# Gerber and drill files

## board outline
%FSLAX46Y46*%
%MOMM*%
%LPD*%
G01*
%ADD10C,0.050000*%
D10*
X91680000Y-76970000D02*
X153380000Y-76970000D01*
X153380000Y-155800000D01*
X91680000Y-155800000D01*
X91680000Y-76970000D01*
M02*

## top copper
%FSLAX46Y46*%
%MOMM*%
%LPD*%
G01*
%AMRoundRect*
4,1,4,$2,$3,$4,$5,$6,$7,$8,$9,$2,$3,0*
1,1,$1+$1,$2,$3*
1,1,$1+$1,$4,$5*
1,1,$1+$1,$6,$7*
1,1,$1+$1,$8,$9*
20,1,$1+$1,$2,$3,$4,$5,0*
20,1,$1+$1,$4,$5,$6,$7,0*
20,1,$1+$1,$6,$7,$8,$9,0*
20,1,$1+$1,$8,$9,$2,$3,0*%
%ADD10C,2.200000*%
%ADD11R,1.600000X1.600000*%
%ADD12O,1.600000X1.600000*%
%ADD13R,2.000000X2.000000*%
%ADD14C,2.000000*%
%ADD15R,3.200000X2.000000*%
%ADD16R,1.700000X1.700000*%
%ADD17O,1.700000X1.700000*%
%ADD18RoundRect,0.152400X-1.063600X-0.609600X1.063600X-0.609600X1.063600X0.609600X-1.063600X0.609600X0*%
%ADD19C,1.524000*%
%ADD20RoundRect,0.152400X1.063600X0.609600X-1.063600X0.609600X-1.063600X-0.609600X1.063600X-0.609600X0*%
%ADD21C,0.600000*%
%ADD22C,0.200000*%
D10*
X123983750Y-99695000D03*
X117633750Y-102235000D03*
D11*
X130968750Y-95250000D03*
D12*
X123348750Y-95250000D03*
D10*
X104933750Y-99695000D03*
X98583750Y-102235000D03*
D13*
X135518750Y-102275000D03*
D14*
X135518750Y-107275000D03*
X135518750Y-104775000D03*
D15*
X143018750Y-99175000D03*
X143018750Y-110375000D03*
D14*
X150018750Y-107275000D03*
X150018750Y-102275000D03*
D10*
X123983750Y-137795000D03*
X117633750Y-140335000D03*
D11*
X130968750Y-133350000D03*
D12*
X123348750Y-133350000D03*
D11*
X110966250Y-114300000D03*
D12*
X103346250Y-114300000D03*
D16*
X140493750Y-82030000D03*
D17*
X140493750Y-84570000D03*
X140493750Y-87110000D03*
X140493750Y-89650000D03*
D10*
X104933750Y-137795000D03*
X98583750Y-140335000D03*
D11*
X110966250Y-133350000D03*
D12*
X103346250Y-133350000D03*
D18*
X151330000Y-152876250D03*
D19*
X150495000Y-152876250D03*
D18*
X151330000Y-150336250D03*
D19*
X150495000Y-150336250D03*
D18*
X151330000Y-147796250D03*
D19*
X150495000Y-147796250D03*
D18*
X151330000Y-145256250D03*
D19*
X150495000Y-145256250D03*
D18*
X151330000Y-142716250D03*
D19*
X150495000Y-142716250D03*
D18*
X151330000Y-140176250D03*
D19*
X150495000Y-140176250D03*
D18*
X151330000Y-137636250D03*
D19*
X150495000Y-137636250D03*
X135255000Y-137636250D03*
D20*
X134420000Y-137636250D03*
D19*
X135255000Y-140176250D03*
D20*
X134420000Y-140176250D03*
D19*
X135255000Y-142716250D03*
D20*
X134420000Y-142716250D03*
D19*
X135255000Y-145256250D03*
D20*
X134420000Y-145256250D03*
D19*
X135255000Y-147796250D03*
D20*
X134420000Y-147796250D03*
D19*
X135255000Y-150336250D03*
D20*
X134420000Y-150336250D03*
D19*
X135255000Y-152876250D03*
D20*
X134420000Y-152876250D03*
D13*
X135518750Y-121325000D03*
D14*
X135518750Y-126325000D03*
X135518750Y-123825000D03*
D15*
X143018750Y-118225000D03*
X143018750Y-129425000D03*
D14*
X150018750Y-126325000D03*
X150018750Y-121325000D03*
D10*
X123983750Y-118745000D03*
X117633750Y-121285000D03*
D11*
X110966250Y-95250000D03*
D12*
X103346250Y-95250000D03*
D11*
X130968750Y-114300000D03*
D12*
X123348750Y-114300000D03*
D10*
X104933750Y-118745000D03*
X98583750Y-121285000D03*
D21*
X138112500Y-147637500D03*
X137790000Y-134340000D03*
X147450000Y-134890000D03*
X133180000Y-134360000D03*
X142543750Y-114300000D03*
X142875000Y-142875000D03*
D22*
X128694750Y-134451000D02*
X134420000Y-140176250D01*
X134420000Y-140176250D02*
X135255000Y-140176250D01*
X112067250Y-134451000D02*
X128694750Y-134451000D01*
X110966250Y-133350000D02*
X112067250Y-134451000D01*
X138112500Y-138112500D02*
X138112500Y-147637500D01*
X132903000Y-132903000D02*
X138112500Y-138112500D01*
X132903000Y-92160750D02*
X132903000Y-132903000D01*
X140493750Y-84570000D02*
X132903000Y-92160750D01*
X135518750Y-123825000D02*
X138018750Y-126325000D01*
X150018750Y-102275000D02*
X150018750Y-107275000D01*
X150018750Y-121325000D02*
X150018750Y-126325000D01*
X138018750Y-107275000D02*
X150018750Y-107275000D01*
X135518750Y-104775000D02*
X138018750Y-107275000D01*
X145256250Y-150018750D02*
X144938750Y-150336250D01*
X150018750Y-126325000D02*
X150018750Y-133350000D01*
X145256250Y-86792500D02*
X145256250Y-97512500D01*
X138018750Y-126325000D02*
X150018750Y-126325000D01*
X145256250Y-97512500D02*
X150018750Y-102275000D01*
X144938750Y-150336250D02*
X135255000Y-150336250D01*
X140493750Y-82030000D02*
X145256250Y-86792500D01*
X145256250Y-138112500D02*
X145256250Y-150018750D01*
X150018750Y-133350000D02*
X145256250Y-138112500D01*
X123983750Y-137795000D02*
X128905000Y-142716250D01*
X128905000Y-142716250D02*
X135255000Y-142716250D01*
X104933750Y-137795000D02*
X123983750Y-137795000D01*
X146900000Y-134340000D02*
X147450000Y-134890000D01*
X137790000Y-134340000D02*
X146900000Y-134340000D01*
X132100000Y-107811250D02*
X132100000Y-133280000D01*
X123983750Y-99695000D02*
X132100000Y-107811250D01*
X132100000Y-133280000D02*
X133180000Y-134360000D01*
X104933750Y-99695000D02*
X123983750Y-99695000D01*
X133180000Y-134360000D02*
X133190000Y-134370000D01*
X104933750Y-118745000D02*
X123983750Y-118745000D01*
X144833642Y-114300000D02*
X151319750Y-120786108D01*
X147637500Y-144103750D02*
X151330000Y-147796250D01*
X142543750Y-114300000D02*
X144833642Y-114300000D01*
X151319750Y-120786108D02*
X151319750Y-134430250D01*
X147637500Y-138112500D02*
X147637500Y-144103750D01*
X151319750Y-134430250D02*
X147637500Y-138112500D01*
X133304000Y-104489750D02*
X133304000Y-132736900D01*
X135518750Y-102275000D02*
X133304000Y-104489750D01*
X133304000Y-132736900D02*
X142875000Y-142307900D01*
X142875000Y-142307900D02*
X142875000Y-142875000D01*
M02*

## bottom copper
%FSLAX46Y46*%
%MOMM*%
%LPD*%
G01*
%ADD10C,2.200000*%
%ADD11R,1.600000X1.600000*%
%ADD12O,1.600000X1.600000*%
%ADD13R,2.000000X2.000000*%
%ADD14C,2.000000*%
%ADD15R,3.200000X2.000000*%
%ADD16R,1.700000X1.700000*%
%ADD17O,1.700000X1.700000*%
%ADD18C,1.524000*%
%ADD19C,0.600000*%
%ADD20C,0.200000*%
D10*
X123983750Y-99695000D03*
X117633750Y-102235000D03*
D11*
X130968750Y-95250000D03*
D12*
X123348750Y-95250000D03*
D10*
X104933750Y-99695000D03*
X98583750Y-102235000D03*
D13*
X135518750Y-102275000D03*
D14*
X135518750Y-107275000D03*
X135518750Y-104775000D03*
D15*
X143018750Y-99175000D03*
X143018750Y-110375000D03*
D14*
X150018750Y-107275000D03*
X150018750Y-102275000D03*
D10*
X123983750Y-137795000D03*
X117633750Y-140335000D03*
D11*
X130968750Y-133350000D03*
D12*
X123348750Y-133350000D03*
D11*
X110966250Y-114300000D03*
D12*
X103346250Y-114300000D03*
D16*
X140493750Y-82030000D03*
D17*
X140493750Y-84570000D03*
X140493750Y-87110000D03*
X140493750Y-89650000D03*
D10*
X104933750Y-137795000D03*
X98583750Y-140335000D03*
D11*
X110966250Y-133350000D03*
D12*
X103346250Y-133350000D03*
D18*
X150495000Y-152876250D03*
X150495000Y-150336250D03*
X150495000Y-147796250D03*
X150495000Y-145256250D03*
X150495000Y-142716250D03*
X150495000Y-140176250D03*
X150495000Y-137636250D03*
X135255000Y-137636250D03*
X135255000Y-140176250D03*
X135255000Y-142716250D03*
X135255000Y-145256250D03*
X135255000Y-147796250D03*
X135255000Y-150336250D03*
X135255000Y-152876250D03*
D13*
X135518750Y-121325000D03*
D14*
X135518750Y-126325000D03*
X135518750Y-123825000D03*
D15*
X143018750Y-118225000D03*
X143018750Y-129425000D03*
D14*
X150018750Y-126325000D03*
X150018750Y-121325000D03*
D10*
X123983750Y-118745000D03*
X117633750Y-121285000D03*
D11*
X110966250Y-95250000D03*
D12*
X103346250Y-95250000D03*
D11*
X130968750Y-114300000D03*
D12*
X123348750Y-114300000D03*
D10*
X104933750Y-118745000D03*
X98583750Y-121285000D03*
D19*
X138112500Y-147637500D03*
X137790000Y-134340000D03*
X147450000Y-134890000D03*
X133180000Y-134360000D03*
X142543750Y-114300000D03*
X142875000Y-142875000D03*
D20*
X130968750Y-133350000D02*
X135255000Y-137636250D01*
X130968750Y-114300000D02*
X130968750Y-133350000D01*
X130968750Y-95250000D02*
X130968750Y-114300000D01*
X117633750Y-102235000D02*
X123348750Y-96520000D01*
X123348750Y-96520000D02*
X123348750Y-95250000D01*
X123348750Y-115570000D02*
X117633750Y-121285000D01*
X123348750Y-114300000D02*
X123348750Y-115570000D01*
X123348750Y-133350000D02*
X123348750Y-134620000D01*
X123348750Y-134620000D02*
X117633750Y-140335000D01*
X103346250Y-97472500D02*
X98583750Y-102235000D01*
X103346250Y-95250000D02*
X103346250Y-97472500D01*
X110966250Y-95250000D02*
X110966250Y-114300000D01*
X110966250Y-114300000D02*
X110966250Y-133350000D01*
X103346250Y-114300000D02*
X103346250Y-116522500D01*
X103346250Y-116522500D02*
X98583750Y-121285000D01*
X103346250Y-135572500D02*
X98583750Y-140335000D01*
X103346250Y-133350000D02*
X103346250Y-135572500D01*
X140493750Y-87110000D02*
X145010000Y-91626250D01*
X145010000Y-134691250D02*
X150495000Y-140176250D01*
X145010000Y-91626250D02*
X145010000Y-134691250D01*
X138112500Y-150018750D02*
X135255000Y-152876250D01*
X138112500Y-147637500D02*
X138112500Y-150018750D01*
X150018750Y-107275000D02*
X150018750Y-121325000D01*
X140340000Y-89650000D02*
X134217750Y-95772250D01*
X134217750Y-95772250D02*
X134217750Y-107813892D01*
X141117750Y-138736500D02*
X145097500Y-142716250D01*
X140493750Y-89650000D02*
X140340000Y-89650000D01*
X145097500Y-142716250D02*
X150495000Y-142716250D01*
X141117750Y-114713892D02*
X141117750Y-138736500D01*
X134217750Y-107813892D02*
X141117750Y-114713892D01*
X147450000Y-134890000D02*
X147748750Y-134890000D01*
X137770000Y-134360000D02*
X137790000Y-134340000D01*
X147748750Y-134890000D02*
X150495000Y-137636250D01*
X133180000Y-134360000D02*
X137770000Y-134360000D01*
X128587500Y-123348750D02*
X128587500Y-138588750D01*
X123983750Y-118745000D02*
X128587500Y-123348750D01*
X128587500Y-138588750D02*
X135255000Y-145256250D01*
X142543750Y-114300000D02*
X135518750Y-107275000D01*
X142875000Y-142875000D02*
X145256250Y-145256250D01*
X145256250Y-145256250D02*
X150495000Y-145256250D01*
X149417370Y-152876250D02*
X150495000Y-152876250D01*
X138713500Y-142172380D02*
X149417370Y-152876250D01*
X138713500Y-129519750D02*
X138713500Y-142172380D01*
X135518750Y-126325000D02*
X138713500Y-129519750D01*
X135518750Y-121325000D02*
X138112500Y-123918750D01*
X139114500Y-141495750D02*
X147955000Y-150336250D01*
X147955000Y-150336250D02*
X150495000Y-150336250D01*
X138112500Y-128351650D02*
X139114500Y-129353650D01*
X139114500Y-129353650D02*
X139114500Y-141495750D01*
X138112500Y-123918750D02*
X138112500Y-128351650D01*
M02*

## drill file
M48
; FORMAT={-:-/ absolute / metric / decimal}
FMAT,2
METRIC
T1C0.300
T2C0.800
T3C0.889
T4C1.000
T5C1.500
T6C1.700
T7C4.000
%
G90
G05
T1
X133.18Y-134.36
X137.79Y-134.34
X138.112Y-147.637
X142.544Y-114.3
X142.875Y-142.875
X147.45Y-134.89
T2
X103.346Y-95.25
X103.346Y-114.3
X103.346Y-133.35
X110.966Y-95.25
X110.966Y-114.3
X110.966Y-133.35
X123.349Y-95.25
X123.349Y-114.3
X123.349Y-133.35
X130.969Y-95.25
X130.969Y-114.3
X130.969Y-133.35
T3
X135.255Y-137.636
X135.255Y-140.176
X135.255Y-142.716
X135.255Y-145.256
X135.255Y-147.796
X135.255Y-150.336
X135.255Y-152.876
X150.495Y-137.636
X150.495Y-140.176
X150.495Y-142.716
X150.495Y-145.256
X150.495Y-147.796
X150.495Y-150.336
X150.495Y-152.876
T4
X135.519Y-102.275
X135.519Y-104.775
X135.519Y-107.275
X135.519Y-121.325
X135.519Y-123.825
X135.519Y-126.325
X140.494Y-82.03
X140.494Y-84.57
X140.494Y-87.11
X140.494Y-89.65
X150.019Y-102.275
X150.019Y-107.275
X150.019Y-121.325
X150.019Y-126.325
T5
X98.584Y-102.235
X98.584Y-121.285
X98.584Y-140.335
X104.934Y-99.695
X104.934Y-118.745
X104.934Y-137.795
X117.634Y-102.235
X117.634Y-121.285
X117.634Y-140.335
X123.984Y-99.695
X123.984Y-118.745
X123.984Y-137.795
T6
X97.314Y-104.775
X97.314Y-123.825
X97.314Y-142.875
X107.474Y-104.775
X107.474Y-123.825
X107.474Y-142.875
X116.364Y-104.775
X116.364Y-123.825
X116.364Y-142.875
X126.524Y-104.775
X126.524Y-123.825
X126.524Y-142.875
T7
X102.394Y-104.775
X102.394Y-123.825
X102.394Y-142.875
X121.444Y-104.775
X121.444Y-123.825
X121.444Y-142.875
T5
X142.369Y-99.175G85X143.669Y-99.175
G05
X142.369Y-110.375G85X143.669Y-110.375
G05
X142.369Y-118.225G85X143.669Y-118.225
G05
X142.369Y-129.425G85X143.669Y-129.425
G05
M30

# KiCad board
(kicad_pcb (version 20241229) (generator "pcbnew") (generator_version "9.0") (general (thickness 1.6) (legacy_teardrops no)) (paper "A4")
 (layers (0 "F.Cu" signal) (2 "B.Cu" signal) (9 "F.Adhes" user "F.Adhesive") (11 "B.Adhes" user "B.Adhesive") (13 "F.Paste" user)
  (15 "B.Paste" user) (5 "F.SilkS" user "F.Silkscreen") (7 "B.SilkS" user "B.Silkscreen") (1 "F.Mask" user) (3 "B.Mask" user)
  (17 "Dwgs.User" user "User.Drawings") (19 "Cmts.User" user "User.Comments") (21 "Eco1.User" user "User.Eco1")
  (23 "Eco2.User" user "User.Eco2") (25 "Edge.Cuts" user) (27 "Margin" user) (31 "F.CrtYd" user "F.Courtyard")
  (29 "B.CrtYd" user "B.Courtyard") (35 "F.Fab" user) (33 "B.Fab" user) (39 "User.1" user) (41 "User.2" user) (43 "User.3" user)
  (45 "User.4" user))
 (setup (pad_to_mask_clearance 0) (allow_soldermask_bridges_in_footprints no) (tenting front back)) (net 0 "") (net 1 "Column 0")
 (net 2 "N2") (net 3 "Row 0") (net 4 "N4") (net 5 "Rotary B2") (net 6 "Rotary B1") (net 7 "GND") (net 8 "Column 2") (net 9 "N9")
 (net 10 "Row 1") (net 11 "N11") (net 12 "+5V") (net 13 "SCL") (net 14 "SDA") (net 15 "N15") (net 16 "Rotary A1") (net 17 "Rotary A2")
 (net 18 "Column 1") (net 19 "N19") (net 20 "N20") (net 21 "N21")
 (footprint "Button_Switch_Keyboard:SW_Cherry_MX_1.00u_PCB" (layer "F.Cu") (at 123.98375 99.695)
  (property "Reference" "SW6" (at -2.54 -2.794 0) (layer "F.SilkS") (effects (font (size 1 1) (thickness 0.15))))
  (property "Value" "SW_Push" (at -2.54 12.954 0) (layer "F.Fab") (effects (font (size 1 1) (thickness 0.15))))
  (pad "" np_thru_hole circle (at -7.62 5.08) (size 1.7 1.7) (drill 1.7) (layers "*.Cu" "*.Mask"))
  (pad "" np_thru_hole circle (at -2.54 5.08) (size 4 4) (drill 4) (layers "*.Cu" "*.Mask"))
  (pad "" np_thru_hole circle (at 2.54 5.08) (size 1.7 1.7) (drill 1.7) (layers "*.Cu" "*.Mask"))
  (pad "1" thru_hole circle (at 0 0) (size 2.2 2.2) (drill 1.5) (layers "*.Cu" "*.Mask") (remove_unused_layers no) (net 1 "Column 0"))
  (pad "2" thru_hole circle (at -6.35 2.54) (size 2.2 2.2) (drill 1.5) (layers "*.Cu" "*.Mask") (remove_unused_layers no) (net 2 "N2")))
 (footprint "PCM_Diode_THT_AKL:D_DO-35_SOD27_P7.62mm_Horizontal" (layer "F.Cu") (at 130.96875 95.25 180)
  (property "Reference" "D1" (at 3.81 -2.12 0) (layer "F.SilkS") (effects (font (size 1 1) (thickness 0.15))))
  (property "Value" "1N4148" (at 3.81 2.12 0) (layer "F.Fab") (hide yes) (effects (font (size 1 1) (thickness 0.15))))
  (pad "1" thru_hole rect (at 0 0 180) (size 1.6 1.6) (drill 0.8) (layers "*.Cu" "*.Mask") (remove_unused_layers no) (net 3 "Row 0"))
  (pad "2" thru_hole oval (at 7.62 0 180) (size 1.6 1.6) (drill 0.8) (layers "*.Cu" "*.Mask") (remove_unused_layers no) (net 2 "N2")))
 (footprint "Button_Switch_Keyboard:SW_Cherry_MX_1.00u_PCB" (layer "F.Cu") (at 104.93375 99.695)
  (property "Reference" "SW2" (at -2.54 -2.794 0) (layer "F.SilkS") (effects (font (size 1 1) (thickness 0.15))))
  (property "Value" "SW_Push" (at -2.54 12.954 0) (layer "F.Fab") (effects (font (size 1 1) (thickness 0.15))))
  (pad "" np_thru_hole circle (at -7.62 5.08) (size 1.7 1.7) (drill 1.7) (layers "*.Cu" "*.Mask"))
  (pad "" np_thru_hole circle (at -2.54 5.08) (size 4 4) (drill 4) (layers "*.Cu" "*.Mask"))
  (pad "" np_thru_hole circle (at 2.54 5.08) (size 1.7 1.7) (drill 1.7) (layers "*.Cu" "*.Mask"))
  (pad "1" thru_hole circle (at 0 0) (size 2.2 2.2) (drill 1.5) (layers "*.Cu" "*.Mask") (remove_unused_layers no) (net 1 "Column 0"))
  (pad "2" thru_hole circle (at -6.35 2.54) (size 2.2 2.2) (drill 1.5) (layers "*.Cu" "*.Mask") (remove_unused_layers no) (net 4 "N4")))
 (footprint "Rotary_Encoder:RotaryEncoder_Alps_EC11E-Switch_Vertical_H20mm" (layer "F.Cu") (at 135.51875 102.275)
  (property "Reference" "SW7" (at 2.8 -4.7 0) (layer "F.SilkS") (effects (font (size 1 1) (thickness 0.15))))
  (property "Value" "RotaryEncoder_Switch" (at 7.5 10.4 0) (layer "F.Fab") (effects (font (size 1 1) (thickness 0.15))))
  (pad "A" thru_hole rect (at 0 0) (size 2 2) (drill 1) (layers "*.Cu" "*.Mask") (remove_unused_layers no) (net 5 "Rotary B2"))
  (pad "B" thru_hole circle (at 0 5) (size 2 2) (drill 1) (layers "*.Cu" "*.Mask") (remove_unused_layers no) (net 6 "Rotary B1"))
  (pad "C" thru_hole circle (at 0 2.5) (size 2 2) (drill 1) (layers "*.Cu" "*.Mask") (remove_unused_layers no) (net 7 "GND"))
  (pad "MP" thru_hole rect (at 7.5 -3.1) (size 3.2 2) (drill oval 2.8 1.5) (layers "*.Cu" "*.Mask") (remove_unused_layers no))
  (pad "MP" thru_hole rect (at 7.5 8.1) (size 3.2 2) (drill oval 2.8 1.5) (layers "*.Cu" "*.Mask") (remove_unused_layers no))
  (pad "S1" thru_hole circle (at 14.5 5) (size 2 2) (drill 1) (layers "*.Cu" "*.Mask") (remove_unused_layers no) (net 7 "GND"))
  (pad "S2" thru_hole circle (at 14.5 0) (size 2 2) (drill 1) (layers "*.Cu" "*.Mask") (remove_unused_layers no) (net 7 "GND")))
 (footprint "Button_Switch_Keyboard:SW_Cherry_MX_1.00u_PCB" (layer "F.Cu") (at 123.98375 137.795)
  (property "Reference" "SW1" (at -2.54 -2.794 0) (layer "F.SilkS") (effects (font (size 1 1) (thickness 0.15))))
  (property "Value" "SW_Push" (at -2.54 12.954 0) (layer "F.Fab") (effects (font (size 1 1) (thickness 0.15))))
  (pad "" np_thru_hole circle (at -7.62 5.08) (size 1.7 1.7) (drill 1.7) (layers "*.Cu" "*.Mask"))
  (pad "" np_thru_hole circle (at -2.54 5.08) (size 4 4) (drill 4) (layers "*.Cu" "*.Mask"))
  (pad "" np_thru_hole circle (at 2.54 5.08) (size 1.7 1.7) (drill 1.7) (layers "*.Cu" "*.Mask"))
  (pad "1" thru_hole circle (at 0 0) (size 2.2 2.2) (drill 1.5) (layers "*.Cu" "*.Mask") (remove_unused_layers no) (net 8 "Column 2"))
  (pad "2" thru_hole circle (at -6.35 2.54) (size 2.2 2.2) (drill 1.5) (layers "*.Cu" "*.Mask") (remove_unused_layers no) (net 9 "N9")))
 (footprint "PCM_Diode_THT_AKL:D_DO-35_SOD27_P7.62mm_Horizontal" (layer "F.Cu") (at 130.96875 133.35 180)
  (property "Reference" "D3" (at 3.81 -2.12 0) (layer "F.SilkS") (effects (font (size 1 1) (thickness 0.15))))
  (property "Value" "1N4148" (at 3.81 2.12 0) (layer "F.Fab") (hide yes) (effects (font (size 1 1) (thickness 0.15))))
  (pad "1" thru_hole rect (at 0 0 180) (size 1.6 1.6) (drill 0.8) (layers "*.Cu" "*.Mask") (remove_unused_layers no) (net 3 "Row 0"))
  (pad "2" thru_hole oval (at 7.62 0 180) (size 1.6 1.6) (drill 0.8) (layers "*.Cu" "*.Mask") (remove_unused_layers no) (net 9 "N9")))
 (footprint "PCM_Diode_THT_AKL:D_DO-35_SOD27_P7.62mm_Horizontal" (layer "F.Cu") (at 110.96625 114.3 180)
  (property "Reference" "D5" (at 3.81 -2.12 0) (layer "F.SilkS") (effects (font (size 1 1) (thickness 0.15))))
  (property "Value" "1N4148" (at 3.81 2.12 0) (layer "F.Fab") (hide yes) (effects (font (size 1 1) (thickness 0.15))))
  (pad "1" thru_hole rect (at 0 0 180) (size 1.6 1.6) (drill 0.8) (layers "*.Cu" "*.Mask") (remove_unused_layers no) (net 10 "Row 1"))
  (pad "2" thru_hole oval (at 7.62 0 180) (size 1.6 1.6) (drill 0.8) (layers "*.Cu" "*.Mask") (remove_unused_layers no) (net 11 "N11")))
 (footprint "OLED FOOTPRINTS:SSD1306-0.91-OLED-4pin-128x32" (layer "F.Cu") (at 103.99375 79.84)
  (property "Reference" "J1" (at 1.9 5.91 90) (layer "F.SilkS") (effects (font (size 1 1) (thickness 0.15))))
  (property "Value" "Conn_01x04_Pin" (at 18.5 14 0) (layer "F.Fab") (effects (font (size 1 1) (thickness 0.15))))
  (pad "1" thru_hole rect (at 36.5 2.19) (size 1.7 1.7) (drill 1) (layers "*.Cu" "*.Mask") (remove_unused_layers no) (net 7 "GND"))
  (pad "2" thru_hole oval (at 36.5 4.73) (size 1.7 1.7) (drill 1) (layers "*.Cu" "*.Mask") (remove_unused_layers no) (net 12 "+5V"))
  (pad "3" thru_hole oval (at 36.5 7.27) (size 1.7 1.7) (drill 1) (layers "*.Cu" "*.Mask") (remove_unused_layers no) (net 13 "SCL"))
  (pad "4" thru_hole oval (at 36.5 9.81) (size 1.7 1.7) (drill 1) (layers "*.Cu" "*.Mask") (remove_unused_layers no) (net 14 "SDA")))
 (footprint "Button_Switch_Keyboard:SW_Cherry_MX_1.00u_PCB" (layer "F.Cu") (at 104.93375 137.795)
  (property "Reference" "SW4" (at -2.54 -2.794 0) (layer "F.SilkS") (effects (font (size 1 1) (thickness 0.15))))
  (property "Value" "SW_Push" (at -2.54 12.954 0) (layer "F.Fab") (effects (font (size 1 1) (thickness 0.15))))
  (pad "" np_thru_hole circle (at -7.62 5.08) (size 1.7 1.7) (drill 1.7) (layers "*.Cu" "*.Mask"))
  (pad "" np_thru_hole circle (at -2.54 5.08) (size 4 4) (drill 4) (layers "*.Cu" "*.Mask"))
  (pad "" np_thru_hole circle (at 2.54 5.08) (size 1.7 1.7) (drill 1.7) (layers "*.Cu" "*.Mask"))
  (pad "1" thru_hole circle (at 0 0) (size 2.2 2.2) (drill 1.5) (layers "*.Cu" "*.Mask") (remove_unused_layers no) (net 8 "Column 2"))
  (pad "2" thru_hole circle (at -6.35 2.54) (size 2.2 2.2) (drill 1.5) (layers "*.Cu" "*.Mask") (remove_unused_layers no) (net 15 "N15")))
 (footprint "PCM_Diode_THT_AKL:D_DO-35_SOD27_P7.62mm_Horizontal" (layer "F.Cu") (at 110.96625 133.35 180)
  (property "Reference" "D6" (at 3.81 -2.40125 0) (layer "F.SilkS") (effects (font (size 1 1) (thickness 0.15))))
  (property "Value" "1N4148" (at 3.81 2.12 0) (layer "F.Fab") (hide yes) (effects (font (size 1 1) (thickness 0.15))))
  (pad "1" thru_hole rect (at 0 0 180) (size 1.6 1.6) (drill 0.8) (layers "*.Cu" "*.Mask") (remove_unused_layers no) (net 10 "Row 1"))
  (pad "2" thru_hole oval (at 7.62 0 180) (size 1.6 1.6) (drill 0.8) (layers "*.Cu" "*.Mask") (remove_unused_layers no) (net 15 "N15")))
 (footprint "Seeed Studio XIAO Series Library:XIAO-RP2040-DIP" (layer "F.Cu") (at 142.875 145.25625 180)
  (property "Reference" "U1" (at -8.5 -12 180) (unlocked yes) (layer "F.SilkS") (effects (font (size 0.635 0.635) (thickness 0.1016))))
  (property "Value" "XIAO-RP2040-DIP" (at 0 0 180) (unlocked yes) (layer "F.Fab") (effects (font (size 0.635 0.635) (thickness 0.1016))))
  (pad "1" smd roundrect (at -8.455 -7.62) (size 2.432 1.524) (layers "F.Cu" "F.Mask") (roundrect_rratio 0.1) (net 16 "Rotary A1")
   (thermal_bridge_angle 45))
  (pad "1" thru_hole circle (at -7.62 -7.62) (size 1.524 1.524) (drill 0.889) (layers "*.Cu" "*.Mask") (remove_unused_layers no)
   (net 16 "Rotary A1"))
  (pad "2" smd roundrect (at -8.455 -5.08) (size 2.432 1.524) (layers "F.Cu" "F.Mask") (roundrect_rratio 0.1) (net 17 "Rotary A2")
   (thermal_bridge_angle 45))
  (pad "2" thru_hole circle (at -7.62 -5.08) (size 1.524 1.524) (drill 0.889) (layers "*.Cu" "*.Mask") (remove_unused_layers no)
   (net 17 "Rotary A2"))
  (pad "3" smd roundrect (at -8.455 -2.54) (size 2.432 1.524) (layers "F.Cu" "F.Mask") (roundrect_rratio 0.1) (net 6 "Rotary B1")
   (thermal_bridge_angle 45))
  (pad "3" thru_hole circle (at -7.62 -2.54) (size 1.524 1.524) (drill 0.889) (layers "*.Cu" "*.Mask") (remove_unused_layers no)
   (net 6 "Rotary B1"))
  (pad "4" smd roundrect (at -8.455 0) (size 2.432 1.524) (layers "F.Cu" "F.Mask") (roundrect_rratio 0.1) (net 5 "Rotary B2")
   (thermal_bridge_angle 45))
  (pad "4" thru_hole circle (at -7.62 0) (size 1.524 1.524) (drill 0.889) (layers "*.Cu" "*.Mask") (remove_unused_layers no)
   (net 5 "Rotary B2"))
  (pad "5" smd roundrect (at -8.455 2.54) (size 2.432 1.524) (layers "F.Cu" "F.Mask") (roundrect_rratio 0.1) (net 14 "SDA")
   (thermal_bridge_angle 45))
  (pad "5" thru_hole circle (at -7.62 2.54) (size 1.524 1.524) (drill 0.889) (layers "*.Cu" "*.Mask") (remove_unused_layers no)
   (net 14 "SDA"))
  (pad "6" smd roundrect (at -8.455 5.08) (size 2.432 1.524) (layers "F.Cu" "F.Mask") (roundrect_rratio 0.1) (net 13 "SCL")
   (thermal_bridge_angle 45))
  (pad "6" thru_hole circle (at -7.62 5.08) (size 1.524 1.524) (drill 0.889) (layers "*.Cu" "*.Mask") (remove_unused_layers no)
   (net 13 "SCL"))
  (pad "7" smd roundrect (at -8.455 7.62) (size 2.432 1.524) (layers "F.Cu" "F.Mask") (roundrect_rratio 0.1) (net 1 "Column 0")
   (thermal_bridge_angle 45))
  (pad "7" thru_hole circle (at -7.62 7.62) (size 1.524 1.524) (drill 0.889) (layers "*.Cu" "*.Mask") (remove_unused_layers no)
   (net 1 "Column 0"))
  (pad "8" thru_hole circle (at 7.62 7.62 180) (size 1.524 1.524) (drill 0.889) (layers "*.Cu" "*.Mask") (remove_unused_layers no)
   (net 3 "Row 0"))
  (pad "8" smd roundrect (at 8.455 7.62 180) (size 2.432 1.524) (layers "F.Cu" "F.Mask") (roundrect_rratio 0.1) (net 3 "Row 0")
   (thermal_bridge_angle 45))
  (pad "9" thru_hole circle (at 7.62 5.08 180) (size 1.524 1.524) (drill 0.889) (layers "*.Cu" "*.Mask") (remove_unused_layers no)
   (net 10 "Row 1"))
  (pad "9" smd roundrect (at 8.455 5.08 180) (size 2.432 1.524) (layers "F.Cu" "F.Mask") (roundrect_rratio 0.1) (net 10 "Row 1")
   (thermal_bridge_angle 45))
  (pad "10" thru_hole circle (at 7.62 2.54 180) (size 1.524 1.524) (drill 0.889) (layers "*.Cu" "*.Mask") (remove_unused_layers no)
   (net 8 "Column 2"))
  (pad "10" smd roundrect (at 8.455 2.54 180) (size 2.432 1.524) (layers "F.Cu" "F.Mask") (roundrect_rratio 0.1) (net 8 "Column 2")
   (thermal_bridge_angle 45))
  (pad "11" thru_hole circle (at 7.62 0 180) (size 1.524 1.524) (drill 0.889) (layers "*.Cu" "*.Mask") (remove_unused_layers no)
   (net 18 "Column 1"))
  (pad "11" smd roundrect (at 8.455 0 180) (size 2.432 1.524) (layers "F.Cu" "F.Mask") (roundrect_rratio 0.1) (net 18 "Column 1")
   (thermal_bridge_angle 45))
  (pad "12" thru_hole circle (at 7.62 -2.54 180) (size 1.524 1.524) (drill 0.889) (layers "*.Cu" "*.Mask") (remove_unused_layers no)
   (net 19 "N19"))
  (pad "12" smd roundrect (at 8.455 -2.54 180) (size 2.432 1.524) (layers "F.Cu" "F.Mask") (roundrect_rratio 0.1) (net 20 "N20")
   (thermal_bridge_angle 45))
  (pad "13" thru_hole circle (at 7.62 -5.08 180) (size 1.524 1.524) (drill 0.889) (layers "*.Cu" "*.Mask") (remove_unused_layers no)
   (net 7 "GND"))
  (pad "13" smd roundrect (at 8.455 -5.08 180) (size 2.432 1.524) (layers "F.Cu" "F.Mask") (roundrect_rratio 0.1) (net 7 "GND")
   (thermal_bridge_angle 45))
  (pad "14" thru_hole circle (at 7.62 -7.62 180) (size 1.524 1.524) (drill 0.889) (layers "*.Cu" "*.Mask") (remove_unused_layers no)
   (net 12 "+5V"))
  (pad "14" smd roundrect (at 8.455 -7.62 180) (size 2.432 1.524) (layers "F.Cu" "F.Mask") (roundrect_rratio 0.1) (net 12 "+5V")
   (thermal_bridge_angle 45)))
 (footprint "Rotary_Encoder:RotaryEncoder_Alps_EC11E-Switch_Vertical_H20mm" (layer "F.Cu") (at 135.51875 121.325)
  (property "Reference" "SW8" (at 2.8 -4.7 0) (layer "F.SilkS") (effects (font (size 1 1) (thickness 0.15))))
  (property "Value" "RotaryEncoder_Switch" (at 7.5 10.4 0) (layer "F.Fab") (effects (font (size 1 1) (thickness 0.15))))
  (pad "A" thru_hole rect (at 0 0) (size 2 2) (drill 1) (layers "*.Cu" "*.Mask") (remove_unused_layers no) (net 17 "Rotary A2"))
  (pad "B" thru_hole circle (at 0 5) (size 2 2) (drill 1) (layers "*.Cu" "*.Mask") (remove_unused_layers no) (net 16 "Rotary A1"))
  (pad "C" thru_hole circle (at 0 2.5) (size 2 2) (drill 1) (layers "*.Cu" "*.Mask") (remove_unused_layers no) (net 7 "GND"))
  (pad "MP" thru_hole rect (at 7.5 -3.1) (size 3.2 2) (drill oval 2.8 1.5) (layers "*.Cu" "*.Mask") (remove_unused_layers no))
  (pad "MP" thru_hole rect (at 7.5 8.1) (size 3.2 2) (drill oval 2.8 1.5) (layers "*.Cu" "*.Mask") (remove_unused_layers no))
  (pad "S1" thru_hole circle (at 14.5 5) (size 2 2) (drill 1) (layers "*.Cu" "*.Mask") (remove_unused_layers no) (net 7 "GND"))
  (pad "S2" thru_hole circle (at 14.5 0) (size 2 2) (drill 1) (layers "*.Cu" "*.Mask") (remove_unused_layers no) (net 7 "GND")))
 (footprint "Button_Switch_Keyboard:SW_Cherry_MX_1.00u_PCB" (layer "F.Cu") (at 123.98375 118.745)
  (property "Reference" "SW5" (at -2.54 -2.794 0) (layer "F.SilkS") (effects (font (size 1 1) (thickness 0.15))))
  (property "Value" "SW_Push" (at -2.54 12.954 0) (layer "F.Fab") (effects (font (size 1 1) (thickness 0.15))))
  (pad "" np_thru_hole circle (at -7.62 5.08) (size 1.7 1.7) (drill 1.7) (layers "*.Cu" "*.Mask"))
  (pad "" np_thru_hole circle (at -2.54 5.08) (size 4 4) (drill 4) (layers "*.Cu" "*.Mask"))
  (pad "" np_thru_hole circle (at 2.54 5.08) (size 1.7 1.7) (drill 1.7) (layers "*.Cu" "*.Mask"))
  (pad "1" thru_hole circle (at 0 0) (size 2.2 2.2) (drill 1.5) (layers "*.Cu" "*.Mask") (remove_unused_layers no) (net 18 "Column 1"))
  (pad "2" thru_hole circle (at -6.35 2.54) (size 2.2 2.2) (drill 1.5) (layers "*.Cu" "*.Mask") (remove_unused_layers no) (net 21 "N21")))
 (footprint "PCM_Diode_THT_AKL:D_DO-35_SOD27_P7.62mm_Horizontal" (layer "F.Cu") (at 110.96625 95.25 180)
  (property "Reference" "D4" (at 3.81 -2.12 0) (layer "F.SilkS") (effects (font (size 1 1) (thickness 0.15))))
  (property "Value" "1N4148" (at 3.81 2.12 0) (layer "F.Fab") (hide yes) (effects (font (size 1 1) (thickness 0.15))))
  (pad "1" thru_hole rect (at 0 0 180) (size 1.6 1.6) (drill 0.8) (layers "*.Cu" "*.Mask") (remove_unused_layers no) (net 10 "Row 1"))
  (pad "2" thru_hole oval (at 7.62 0 180) (size 1.6 1.6) (drill 0.8) (layers "*.Cu" "*.Mask") (remove_unused_layers no) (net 4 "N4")))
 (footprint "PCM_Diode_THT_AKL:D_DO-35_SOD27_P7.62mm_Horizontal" (layer "F.Cu") (at 130.96875 114.3 180)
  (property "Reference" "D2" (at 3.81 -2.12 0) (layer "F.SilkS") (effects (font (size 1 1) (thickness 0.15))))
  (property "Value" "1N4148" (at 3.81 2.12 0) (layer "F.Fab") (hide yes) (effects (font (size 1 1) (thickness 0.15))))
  (pad "1" thru_hole rect (at 0 0 180) (size 1.6 1.6) (drill 0.8) (layers "*.Cu" "*.Mask") (remove_unused_layers no) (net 3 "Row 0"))
  (pad "2" thru_hole oval (at 7.62 0 180) (size 1.6 1.6) (drill 0.8) (layers "*.Cu" "*.Mask") (remove_unused_layers no) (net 21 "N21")))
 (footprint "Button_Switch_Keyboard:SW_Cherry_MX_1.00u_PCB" (layer "F.Cu") (at 104.93375 118.745)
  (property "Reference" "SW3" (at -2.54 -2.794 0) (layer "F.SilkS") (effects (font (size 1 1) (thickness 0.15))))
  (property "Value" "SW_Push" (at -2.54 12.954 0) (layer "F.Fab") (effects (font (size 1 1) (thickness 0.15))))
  (pad "" np_thru_hole circle (at -7.62 5.08) (size 1.7 1.7) (drill 1.7) (layers "*.Cu" "*.Mask"))
  (pad "" np_thru_hole circle (at -2.54 5.08) (size 4 4) (drill 4) (layers "*.Cu" "*.Mask"))
  (pad "" np_thru_hole circle (at 2.54 5.08) (size 1.7 1.7) (drill 1.7) (layers "*.Cu" "*.Mask"))
  (pad "1" thru_hole circle (at 0 0) (size 2.2 2.2) (drill 1.5) (layers "*.Cu" "*.Mask") (remove_unused_layers no) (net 18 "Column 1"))
  (pad "2" thru_hole circle (at -6.35 2.54) (size 2.2 2.2) (drill 1.5) (layers "*.Cu" "*.Mask") (remove_unused_layers no) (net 11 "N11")))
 (gr_rect (start 91.68 76.97) (end 153.38 155.8) (stroke (width 0.05) (type default)) (fill no) (layer "Edge.Cuts"))
 (segment (start 130.96875 133.35) (end 135.255 137.63625) (width 0.2) (layer "B.Cu") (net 3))
 (segment (start 130.96875 114.3) (end 130.96875 133.35) (width 0.2) (layer "B.Cu") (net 3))
 (segment (start 130.96875 95.25) (end 130.96875 114.3) (width 0.2) (layer "B.Cu") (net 3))
 (segment (start 117.63375 102.235) (end 123.34875 96.52) (width 0.2) (layer "B.Cu") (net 2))
 (segment (start 123.34875 96.52) (end 123.34875 95.25) (width 0.2) (layer "B.Cu") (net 2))
 (segment (start 123.34875 115.57) (end 117.63375 121.285) (width 0.2) (layer "B.Cu") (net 21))
 (segment (start 123.34875 114.3) (end 123.34875 115.57) (width 0.2) (layer "B.Cu") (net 21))
 (segment (start 123.34875 133.35) (end 123.34875 134.62) (width 0.2) (layer "B.Cu") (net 9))
 (segment (start 123.34875 134.62) (end 117.63375 140.335) (width 0.2) (layer "B.Cu") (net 9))
 (segment (start 103.34625 97.4725) (end 98.58375 102.235) (width 0.2) (layer "B.Cu") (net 4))
 (segment (start 103.34625 95.25) (end 103.34625 97.4725) (width 0.2) (layer "B.Cu") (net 4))
 (segment (start 128.69475 134.451) (end 134.42 140.17625) (width 0.2) (layer "F.Cu") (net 10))
 (segment (start 134.42 140.17625) (end 135.255 140.17625) (width 0.2) (layer "F.Cu") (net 10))
 (segment (start 112.06725 134.451) (end 128.69475 134.451) (width 0.2) (layer "F.Cu") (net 10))
 (segment (start 110.96625 133.35) (end 112.06725 134.451) (width 0.2) (layer "F.Cu") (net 10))
 (segment (start 110.96625 95.25) (end 110.96625 114.3) (width 0.2) (layer "B.Cu") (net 10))
 (segment (start 110.96625 114.3) (end 110.96625 133.35) (width 0.2) (layer "B.Cu") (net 10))
 (segment (start 103.34625 114.3) (end 103.34625 116.5225) (width 0.2) (layer "B.Cu") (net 11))
 (segment (start 103.34625 116.5225) (end 98.58375 121.285) (width 0.2) (layer "B.Cu") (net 11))
 (segment (start 103.34625 135.5725) (end 98.58375 140.335) (width 0.2) (layer "B.Cu") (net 15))
 (segment (start 103.34625 133.35) (end 103.34625 135.5725) (width 0.2) (layer "B.Cu") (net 15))
 (segment (start 140.49375 87.11) (end 145.01 91.62625) (width 0.2) (layer "B.Cu") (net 13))
 (segment (start 145.01 134.69125) (end 150.495 140.17625) (width 0.2) (layer "B.Cu") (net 13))
 (segment (start 145.01 91.62625) (end 145.01 134.69125) (width 0.2) (layer "B.Cu") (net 13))
 (segment (start 138.1125 138.1125) (end 138.1125 147.6375) (width 0.2) (layer "F.Cu") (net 12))
 (segment (start 132.903 132.903) (end 138.1125 138.1125) (width 0.2) (layer "F.Cu") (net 12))
 (segment (start 132.903 92.16075) (end 132.903 132.903) (width 0.2) (layer "F.Cu") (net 12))
 (segment (start 140.49375 84.57) (end 132.903 92.16075) (width 0.2) (layer "F.Cu") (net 12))
 (via (at 138.1125 147.6375) (size 0.6) (drill 0.3) (layers "F.Cu" "B.Cu") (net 12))
 (segment (start 138.1125 150.01875) (end 135.255 152.87625) (width 0.2) (layer "B.Cu") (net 12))
 (segment (start 138.1125 147.6375) (end 138.1125 150.01875) (width 0.2) (layer "B.Cu") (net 12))
 (segment (start 135.51875 123.825) (end 138.01875 126.325) (width 0.2) (layer "F.Cu") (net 7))
 (segment (start 150.01875 102.275) (end 150.01875 107.275) (width 0.2) (layer "F.Cu") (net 7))
 (segment (start 150.01875 121.325) (end 150.01875 126.325) (width 0.2) (layer "F.Cu") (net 7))
 (segment (start 138.01875 107.275) (end 150.01875 107.275) (width 0.2) (layer "F.Cu") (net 7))
 (segment (start 135.51875 104.775) (end 138.01875 107.275) (width 0.2) (layer "F.Cu") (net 7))
 (segment (start 145.25625 150.01875) (end 144.93875 150.33625) (width 0.2) (layer "F.Cu") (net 7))
 (segment (start 150.01875 126.325) (end 150.01875 133.35) (width 0.2) (layer "F.Cu") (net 7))
 (segment (start 145.25625 86.7925) (end 145.25625 97.5125) (width 0.2) (layer "F.Cu") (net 7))
 (segment (start 138.01875 126.325) (end 150.01875 126.325) (width 0.2) (layer "F.Cu") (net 7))
 (segment (start 145.25625 97.5125) (end 150.01875 102.275) (width 0.2) (layer "F.Cu") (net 7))
 (segment (start 144.93875 150.33625) (end 135.255 150.33625) (width 0.2) (layer "F.Cu") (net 7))
 (segment (start 140.49375 82.03) (end 145.25625 86.7925) (width 0.2) (layer "F.Cu") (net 7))
 (segment (start 145.25625 138.1125) (end 145.25625 150.01875) (width 0.2) (layer "F.Cu") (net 7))
 (segment (start 150.01875 133.35) (end 145.25625 138.1125) (width 0.2) (layer "F.Cu") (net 7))
 (segment (start 150.01875 107.275) (end 150.01875 121.325) (width 0.2) (layer "B.Cu") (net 7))
 (segment (start 140.34 89.65) (end 134.21775 95.77225) (width 0.2) (layer "B.Cu") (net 14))
 (segment (start 134.21775 95.77225) (end 134.21775 107.813892) (width 0.2) (layer "B.Cu") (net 14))
 (segment (start 141.11775 138.7365) (end 145.0975 142.71625) (width 0.2) (layer "B.Cu") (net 14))
 (segment (start 140.49375 89.65) (end 140.34 89.65) (width 0.2) (layer "B.Cu") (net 14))
 (segment (start 145.0975 142.71625) (end 150.495 142.71625) (width 0.2) (layer "B.Cu") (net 14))
 (segment (start 141.11775 114.713892) (end 141.11775 138.7365) (width 0.2) (layer "B.Cu") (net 14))
 (segment (start 134.21775 107.813892) (end 141.11775 114.713892) (width 0.2) (layer "B.Cu") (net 14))
 (segment (start 123.98375 137.795) (end 128.905 142.71625) (width 0.2) (layer "F.Cu") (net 8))
 (segment (start 128.905 142.71625) (end 135.255 142.71625) (width 0.2) (layer "F.Cu") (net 8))
 (segment (start 104.93375 137.795) (end 123.98375 137.795) (width 0.2) (layer "F.Cu") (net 8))
 (segment (start 146.9 134.34) (end 147.45 134.89) (width 0.2) (layer "F.Cu") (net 1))
 (segment (start 137.79 134.34) (end 146.9 134.34) (width 0.2) (layer "F.Cu") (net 1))
 (segment (start 132.1 107.81125) (end 132.1 133.28) (width 0.2) (layer "F.Cu") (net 1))
 (segment (start 123.98375 99.695) (end 132.1 107.81125) (width 0.2) (layer "F.Cu") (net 1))
 (segment (start 132.1 133.28) (end 133.18 134.36) (width 0.2) (layer "F.Cu") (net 1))
 (segment (start 104.93375 99.695) (end 123.98375 99.695) (width 0.2) (layer "F.Cu") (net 1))
 (segment (start 133.18 134.36) (end 133.19 134.37) (width 0.2) (layer "F.Cu") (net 1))
 (via (at 137.79 134.34) (size 0.6) (drill 0.3) (layers "F.Cu" "B.Cu") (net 1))
 (via (at 147.45 134.89) (size 0.6) (drill 0.3) (layers "F.Cu" "B.Cu") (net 1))
 (via (at 133.18 134.36) (size 0.6) (drill 0.3) (layers "F.Cu" "B.Cu") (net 1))
 (segment (start 147.45 134.89) (end 147.74875 134.89) (width 0.2) (layer "B.Cu") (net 1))
 (segment (start 137.77 134.36) (end 137.79 134.34) (width 0.2) (layer "B.Cu") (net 1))
 (segment (start 147.74875 134.89) (end 150.495 137.63625) (width 0.2) (layer "B.Cu") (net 1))
 (segment (start 133.18 134.36) (end 137.77 134.36) (width 0.2) (layer "B.Cu") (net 1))
 (segment (start 104.93375 118.745) (end 123.98375 118.745) (width 0.2) (layer "F.Cu") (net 18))
 (segment (start 128.5875 123.34875) (end 128.5875 138.58875) (width 0.2) (layer "B.Cu") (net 18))
 (segment (start 123.98375 118.745) (end 128.5875 123.34875) (width 0.2) (layer "B.Cu") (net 18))
 (segment (start 128.5875 138.58875) (end 135.255 145.25625) (width 0.2) (layer "B.Cu") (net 18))
 (segment (start 144.833642 114.3) (end 151.31975 120.786108) (width 0.2) (layer "F.Cu") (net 6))
 (segment (start 147.6375 144.10375) (end 151.33 147.79625) (width 0.2) (layer "F.Cu") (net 6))
 (segment (start 142.54375 114.3) (end 144.833642 114.3) (width 0.2) (layer "F.Cu") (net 6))
 (segment (start 151.31975 120.786108) (end 151.31975 134.43025) (width 0.2) (layer "F.Cu") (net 6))
 (segment (start 147.6375 138.1125) (end 147.6375 144.10375) (width 0.2) (layer "F.Cu") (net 6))
 (segment (start 151.31975 134.43025) (end 147.6375 138.1125) (width 0.2) (layer "F.Cu") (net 6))
 (via (at 142.54375 114.3) (size 0.6) (drill 0.3) (layers "F.Cu" "B.Cu") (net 6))
 (segment (start 142.54375 114.3) (end 135.51875 107.275) (width 0.2) (layer "B.Cu") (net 6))
 (segment (start 133.304 104.48975) (end 133.304 132.7369) (width 0.2) (layer "F.Cu") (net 5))
 (segment (start 135.51875 102.275) (end 133.304 104.48975) (width 0.2) (layer "F.Cu") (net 5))
 (segment (start 133.304 132.7369) (end 142.875 142.3079) (width 0.2) (layer "F.Cu") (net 5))
 (segment (start 142.875 142.3079) (end 142.875 142.875) (width 0.2) (layer "F.Cu") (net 5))
 (via (at 142.875 142.875) (size 0.6) (drill 0.3) (layers "F.Cu" "B.Cu") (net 5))
 (segment (start 142.875 142.875) (end 145.25625 145.25625) (width 0.2) (layer "B.Cu") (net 5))
 (segment (start 145.25625 145.25625) (end 150.495 145.25625) (width 0.2) (layer "B.Cu") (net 5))
 (segment (start 149.41737 152.87625) (end 150.495 152.87625) (width 0.2) (layer "B.Cu") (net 16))
 (segment (start 138.7135 142.17238) (end 149.41737 152.87625) (width 0.2) (layer "B.Cu") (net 16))
 (segment (start 138.7135 129.51975) (end 138.7135 142.17238) (width 0.2) (layer "B.Cu") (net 16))
 (segment (start 135.51875 126.325) (end 138.7135 129.51975) (width 0.2) (layer "B.Cu") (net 16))
 (segment (start 135.51875 121.325) (end 138.1125 123.91875) (width 0.2) (layer "B.Cu") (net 17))
 (segment (start 139.1145 141.49575) (end 147.955 150.33625) (width 0.2) (layer "B.Cu") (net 17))
 (segment (start 147.955 150.33625) (end 150.495 150.33625) (width 0.2) (layer "B.Cu") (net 17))
 (segment (start 138.1125 128.35165) (end 139.1145 129.35365) (width 0.2) (layer "B.Cu") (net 17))
 (segment (start 139.1145 129.35365) (end 139.1145 141.49575) (width 0.2) (layer "B.Cu") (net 17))
 (segment (start 138.1125 123.91875) (end 138.1125 128.35165) (width 0.2) (layer "B.Cu") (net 17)))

